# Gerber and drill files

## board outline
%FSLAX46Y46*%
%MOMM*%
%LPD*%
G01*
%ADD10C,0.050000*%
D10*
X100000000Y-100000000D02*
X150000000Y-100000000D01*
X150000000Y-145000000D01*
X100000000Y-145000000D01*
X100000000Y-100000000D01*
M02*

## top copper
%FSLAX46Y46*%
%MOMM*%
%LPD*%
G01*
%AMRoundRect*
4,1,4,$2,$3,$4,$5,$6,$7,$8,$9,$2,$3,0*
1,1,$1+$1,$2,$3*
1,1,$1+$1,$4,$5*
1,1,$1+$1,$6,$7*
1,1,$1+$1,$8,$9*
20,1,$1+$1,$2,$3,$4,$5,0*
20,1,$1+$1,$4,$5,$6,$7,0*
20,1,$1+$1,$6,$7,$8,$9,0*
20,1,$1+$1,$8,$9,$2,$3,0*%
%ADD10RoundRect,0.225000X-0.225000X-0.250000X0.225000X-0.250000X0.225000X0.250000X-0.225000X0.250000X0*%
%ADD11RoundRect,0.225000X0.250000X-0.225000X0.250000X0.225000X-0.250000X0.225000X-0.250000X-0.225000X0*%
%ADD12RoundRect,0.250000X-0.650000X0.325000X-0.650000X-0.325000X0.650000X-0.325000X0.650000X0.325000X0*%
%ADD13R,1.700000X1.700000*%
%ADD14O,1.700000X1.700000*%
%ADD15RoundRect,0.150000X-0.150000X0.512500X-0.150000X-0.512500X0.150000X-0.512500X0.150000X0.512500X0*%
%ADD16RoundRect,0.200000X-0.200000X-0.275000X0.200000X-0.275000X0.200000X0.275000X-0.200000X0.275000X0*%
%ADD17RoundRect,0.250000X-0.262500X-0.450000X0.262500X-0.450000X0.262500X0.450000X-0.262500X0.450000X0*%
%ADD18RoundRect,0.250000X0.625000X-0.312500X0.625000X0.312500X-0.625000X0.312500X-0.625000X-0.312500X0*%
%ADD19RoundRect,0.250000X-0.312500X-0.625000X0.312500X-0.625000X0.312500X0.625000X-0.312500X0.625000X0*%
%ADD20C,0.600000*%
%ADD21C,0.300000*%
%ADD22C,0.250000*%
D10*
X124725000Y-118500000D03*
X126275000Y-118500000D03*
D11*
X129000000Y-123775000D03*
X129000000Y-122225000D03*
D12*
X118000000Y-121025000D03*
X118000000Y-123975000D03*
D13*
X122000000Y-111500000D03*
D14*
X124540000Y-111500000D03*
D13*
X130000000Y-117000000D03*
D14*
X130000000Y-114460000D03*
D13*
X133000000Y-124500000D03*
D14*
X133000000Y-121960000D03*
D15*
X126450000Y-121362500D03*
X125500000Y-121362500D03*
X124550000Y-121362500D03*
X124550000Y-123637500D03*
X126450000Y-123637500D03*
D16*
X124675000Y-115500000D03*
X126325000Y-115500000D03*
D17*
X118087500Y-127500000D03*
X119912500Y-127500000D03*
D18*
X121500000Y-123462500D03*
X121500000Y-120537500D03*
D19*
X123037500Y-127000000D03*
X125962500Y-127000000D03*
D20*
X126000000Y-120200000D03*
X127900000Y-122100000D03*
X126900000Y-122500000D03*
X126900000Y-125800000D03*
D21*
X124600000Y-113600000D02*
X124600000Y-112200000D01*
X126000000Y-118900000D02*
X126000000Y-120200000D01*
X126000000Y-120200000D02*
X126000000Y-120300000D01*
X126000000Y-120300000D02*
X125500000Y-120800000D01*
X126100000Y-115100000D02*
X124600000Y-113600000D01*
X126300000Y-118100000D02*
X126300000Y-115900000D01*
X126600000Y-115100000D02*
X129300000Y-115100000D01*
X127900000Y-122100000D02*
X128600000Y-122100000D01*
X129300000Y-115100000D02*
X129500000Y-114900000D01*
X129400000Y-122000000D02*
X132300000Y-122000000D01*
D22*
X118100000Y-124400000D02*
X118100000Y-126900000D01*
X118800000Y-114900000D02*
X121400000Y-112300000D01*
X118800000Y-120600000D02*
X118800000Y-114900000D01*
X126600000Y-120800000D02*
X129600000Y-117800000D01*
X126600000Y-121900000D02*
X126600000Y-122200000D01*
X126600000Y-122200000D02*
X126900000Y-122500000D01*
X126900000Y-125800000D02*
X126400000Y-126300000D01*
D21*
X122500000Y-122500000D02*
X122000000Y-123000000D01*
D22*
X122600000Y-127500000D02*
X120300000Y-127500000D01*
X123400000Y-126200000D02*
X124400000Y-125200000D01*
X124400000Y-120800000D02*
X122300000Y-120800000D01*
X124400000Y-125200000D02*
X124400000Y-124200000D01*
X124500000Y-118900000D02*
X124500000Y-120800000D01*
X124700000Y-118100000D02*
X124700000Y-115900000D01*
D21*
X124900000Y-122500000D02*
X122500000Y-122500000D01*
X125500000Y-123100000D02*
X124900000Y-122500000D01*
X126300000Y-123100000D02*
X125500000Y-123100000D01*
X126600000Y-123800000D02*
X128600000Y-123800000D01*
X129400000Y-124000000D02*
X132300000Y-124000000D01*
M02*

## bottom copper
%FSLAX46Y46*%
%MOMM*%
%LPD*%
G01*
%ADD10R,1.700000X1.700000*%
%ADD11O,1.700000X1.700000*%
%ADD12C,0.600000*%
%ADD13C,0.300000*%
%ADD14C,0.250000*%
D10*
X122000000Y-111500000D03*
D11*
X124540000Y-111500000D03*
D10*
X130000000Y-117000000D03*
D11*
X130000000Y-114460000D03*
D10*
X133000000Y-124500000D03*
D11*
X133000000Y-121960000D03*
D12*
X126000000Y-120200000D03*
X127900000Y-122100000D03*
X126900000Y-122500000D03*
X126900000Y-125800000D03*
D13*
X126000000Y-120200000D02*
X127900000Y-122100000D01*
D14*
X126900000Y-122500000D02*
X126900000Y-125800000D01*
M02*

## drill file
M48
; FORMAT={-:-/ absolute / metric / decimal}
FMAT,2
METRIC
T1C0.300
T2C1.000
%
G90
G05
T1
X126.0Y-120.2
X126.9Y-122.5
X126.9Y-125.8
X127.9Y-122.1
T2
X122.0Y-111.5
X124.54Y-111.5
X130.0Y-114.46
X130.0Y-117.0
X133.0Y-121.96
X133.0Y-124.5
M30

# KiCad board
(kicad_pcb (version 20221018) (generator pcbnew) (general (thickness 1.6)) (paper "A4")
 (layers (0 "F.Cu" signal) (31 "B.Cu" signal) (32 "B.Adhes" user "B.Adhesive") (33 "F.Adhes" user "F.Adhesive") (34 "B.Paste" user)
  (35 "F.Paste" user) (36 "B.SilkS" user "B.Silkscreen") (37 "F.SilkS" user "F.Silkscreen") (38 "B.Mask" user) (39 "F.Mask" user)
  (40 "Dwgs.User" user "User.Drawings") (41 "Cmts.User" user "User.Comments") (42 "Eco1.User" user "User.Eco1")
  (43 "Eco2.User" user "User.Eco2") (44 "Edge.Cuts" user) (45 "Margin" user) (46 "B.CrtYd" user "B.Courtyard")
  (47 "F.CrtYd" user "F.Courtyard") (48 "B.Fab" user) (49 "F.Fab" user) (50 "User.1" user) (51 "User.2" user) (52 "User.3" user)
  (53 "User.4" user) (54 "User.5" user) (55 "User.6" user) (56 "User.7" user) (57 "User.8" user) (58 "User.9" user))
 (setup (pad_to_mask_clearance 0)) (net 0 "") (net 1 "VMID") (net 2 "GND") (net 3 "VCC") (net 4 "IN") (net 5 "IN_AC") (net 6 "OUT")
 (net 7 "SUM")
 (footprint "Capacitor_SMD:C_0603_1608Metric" (layer "F.Cu") (at 125.5 118.5)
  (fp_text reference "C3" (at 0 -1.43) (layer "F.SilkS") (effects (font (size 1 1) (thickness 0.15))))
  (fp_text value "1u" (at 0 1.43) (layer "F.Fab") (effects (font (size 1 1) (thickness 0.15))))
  (pad "1" smd roundrect (at -0.775 0) (size 0.9 0.95) (layers "F.Cu" "F.Paste" "F.Mask") (roundrect_rratio 0.25) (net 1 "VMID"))
  (pad "2" smd roundrect (at 0.775 0) (size 0.9 0.95) (layers "F.Cu" "F.Paste" "F.Mask") (roundrect_rratio 0.25) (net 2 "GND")))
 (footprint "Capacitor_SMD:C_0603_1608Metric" (layer "F.Cu") (at 129 123 90)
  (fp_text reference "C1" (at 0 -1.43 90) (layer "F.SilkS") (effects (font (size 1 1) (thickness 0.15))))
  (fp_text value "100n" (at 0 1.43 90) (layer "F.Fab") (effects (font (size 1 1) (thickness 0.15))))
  (pad "1" smd roundrect (at -0.775 0 90) (size 0.9 0.95) (layers "F.Cu" "F.Paste" "F.Mask") (roundrect_rratio 0.25) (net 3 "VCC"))
  (pad "2" smd roundrect (at 0.775 0 90) (size 0.9 0.95) (layers "F.Cu" "F.Paste" "F.Mask") (roundrect_rratio 0.25) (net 2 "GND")))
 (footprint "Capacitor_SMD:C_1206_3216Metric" (layer "F.Cu") (at 118 122.5 -90)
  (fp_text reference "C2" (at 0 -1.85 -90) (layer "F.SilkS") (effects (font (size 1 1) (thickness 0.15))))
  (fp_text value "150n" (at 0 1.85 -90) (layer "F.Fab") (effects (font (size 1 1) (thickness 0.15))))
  (pad "1" smd roundrect (at -1.475 0 270) (size 1.15 1.8) (layers "F.Cu" "F.Paste" "F.Mask") (roundrect_rratio 0.217391) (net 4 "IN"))
  (pad "2" smd roundrect (at 1.475 0 270) (size 1.15 1.8) (layers "F.Cu" "F.Paste" "F.Mask") (roundrect_rratio 0.217391) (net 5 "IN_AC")))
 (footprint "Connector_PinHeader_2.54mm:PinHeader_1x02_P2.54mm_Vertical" (layer "F.Cu") (at 122 111.5 90)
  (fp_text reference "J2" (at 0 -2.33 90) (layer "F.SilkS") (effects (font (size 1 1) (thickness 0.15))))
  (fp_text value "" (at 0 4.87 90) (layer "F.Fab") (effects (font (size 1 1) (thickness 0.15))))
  (pad "1" thru_hole rect (at 0 0 90) (size 1.7 1.7) (drill 1) (layers "*.Cu" "*.Mask") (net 4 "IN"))
  (pad "2" thru_hole oval (at 0 2.54 90) (size 1.7 1.7) (drill 1) (layers "*.Cu" "*.Mask") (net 2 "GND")))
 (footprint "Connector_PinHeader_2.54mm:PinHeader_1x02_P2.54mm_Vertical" (layer "F.Cu") (at 130 117 180)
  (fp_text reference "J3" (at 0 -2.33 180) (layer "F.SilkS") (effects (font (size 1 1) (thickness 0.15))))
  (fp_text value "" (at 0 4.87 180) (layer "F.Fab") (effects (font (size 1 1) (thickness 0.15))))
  (pad "1" thru_hole rect (at 0 0 180) (size 1.7 1.7) (drill 1) (layers "*.Cu" "*.Mask") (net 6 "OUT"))
  (pad "2" thru_hole oval (at 0 2.54 180) (size 1.7 1.7) (drill 1) (layers "*.Cu" "*.Mask") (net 2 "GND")))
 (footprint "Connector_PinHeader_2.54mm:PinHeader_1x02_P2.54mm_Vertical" (layer "F.Cu") (at 133 124.5 180)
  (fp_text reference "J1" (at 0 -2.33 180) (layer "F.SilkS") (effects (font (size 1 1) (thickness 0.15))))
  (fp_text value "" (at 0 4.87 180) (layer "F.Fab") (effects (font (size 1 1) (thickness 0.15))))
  (pad "1" thru_hole rect (at 0 0 180) (size 1.7 1.7) (drill 1) (layers "*.Cu" "*.Mask") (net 3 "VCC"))
  (pad "2" thru_hole oval (at 0 2.54 180) (size 1.7 1.7) (drill 1) (layers "*.Cu" "*.Mask") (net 2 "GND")))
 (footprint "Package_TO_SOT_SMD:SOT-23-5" (layer "F.Cu") (at 125.5 122.5 -90)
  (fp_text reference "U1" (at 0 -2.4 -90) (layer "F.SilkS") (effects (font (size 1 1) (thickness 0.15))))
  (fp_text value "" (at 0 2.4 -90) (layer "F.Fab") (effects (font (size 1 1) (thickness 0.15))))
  (pad "1" smd roundrect (at -1.1375 -0.95 270) (size 1.325 0.6) (layers "F.Cu" "F.Paste" "F.Mask") (roundrect_rratio 0.25) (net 6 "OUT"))
  (pad "2" smd roundrect (at -1.1375 0 270) (size 1.325 0.6) (layers "F.Cu" "F.Paste" "F.Mask") (roundrect_rratio 0.25) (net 2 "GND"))
  (pad "3" smd roundrect (at -1.1375 0.95 270) (size 1.325 0.6) (layers "F.Cu" "F.Paste" "F.Mask") (roundrect_rratio 0.25) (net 1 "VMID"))
  (pad "4" smd roundrect (at 1.1375 0.95 270) (size 1.325 0.6) (layers "F.Cu" "F.Paste" "F.Mask") (roundrect_rratio 0.25) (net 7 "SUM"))
  (pad "5" smd roundrect (at 1.1375 -0.95 270) (size 1.325 0.6) (layers "F.Cu" "F.Paste" "F.Mask") (roundrect_rratio 0.25) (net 3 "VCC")))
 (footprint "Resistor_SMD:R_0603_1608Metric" (layer "F.Cu") (at 125.5 115.5)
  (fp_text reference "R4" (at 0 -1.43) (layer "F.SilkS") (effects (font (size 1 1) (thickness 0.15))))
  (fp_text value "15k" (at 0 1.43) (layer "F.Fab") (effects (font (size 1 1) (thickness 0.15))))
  (pad "1" smd roundrect (at -0.825 0) (size 0.8 0.95) (layers "F.Cu" "F.Paste" "F.Mask") (roundrect_rratio 0.25) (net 1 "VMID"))
  (pad "2" smd roundrect (at 0.825 0) (size 0.8 0.95) (layers "F.Cu" "F.Paste" "F.Mask") (roundrect_rratio 0.25) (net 2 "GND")))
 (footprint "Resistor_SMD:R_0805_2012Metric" (layer "F.Cu") (at 119 127.5)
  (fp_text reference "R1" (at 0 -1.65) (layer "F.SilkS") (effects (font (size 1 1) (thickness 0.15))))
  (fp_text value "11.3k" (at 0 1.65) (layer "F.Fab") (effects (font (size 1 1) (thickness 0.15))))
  (pad "1" smd roundrect (at -0.9125 0) (size 1.025 1.4) (layers "F.Cu" "F.Paste" "F.Mask") (roundrect_rratio 0.243902) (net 5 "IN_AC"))
  (pad "2" smd roundrect (at 0.9125 0) (size 1.025 1.4) (layers "F.Cu" "F.Paste" "F.Mask") (roundrect_rratio 0.243902) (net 7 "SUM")))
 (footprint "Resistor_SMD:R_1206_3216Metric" (layer "F.Cu") (at 121.5 122 90)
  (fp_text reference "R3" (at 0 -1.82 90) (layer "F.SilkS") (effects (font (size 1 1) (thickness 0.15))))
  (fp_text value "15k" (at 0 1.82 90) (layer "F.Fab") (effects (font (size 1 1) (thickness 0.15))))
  (pad "1" smd roundrect (at -1.4625 0 90) (size 1.125 1.75) (layers "F.Cu" "F.Paste" "F.Mask") (roundrect_rratio 0.222222) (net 3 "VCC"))
  (pad "2" smd roundrect (at 1.4625 0 90) (size 1.125 1.75) (layers "F.Cu" "F.Paste" "F.Mask") (roundrect_rratio 0.222222) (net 1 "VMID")))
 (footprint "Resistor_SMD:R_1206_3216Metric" (layer "F.Cu") (at 124.5 127)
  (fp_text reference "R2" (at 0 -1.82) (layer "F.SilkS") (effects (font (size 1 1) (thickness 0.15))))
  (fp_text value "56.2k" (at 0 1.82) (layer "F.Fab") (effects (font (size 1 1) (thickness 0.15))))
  (pad "1" smd roundrect (at -1.4625 0) (size 1.125 1.75) (layers "F.Cu" "F.Paste" "F.Mask") (roundrect_rratio 0.222222) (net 7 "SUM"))
  (pad "2" smd roundrect (at 1.4625 0) (size 1.125 1.75) (layers "F.Cu" "F.Paste" "F.Mask") (roundrect_rratio 0.222222) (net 6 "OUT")))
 (gr_rect (start 100 100) (end 150 145) (stroke (width 0.05) (type default)) (fill none) (layer "Edge.Cuts"))
 (segment (start 124.6 113.6) (end 124.6 112.2) (width 0.3) (layer "F.Cu") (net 2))
 (segment (start 126 118.9) (end 126 120.2) (width 0.3) (layer "F.Cu") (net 2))
 (segment (start 126 120.2) (end 126 120.3) (width 0.3) (layer "F.Cu") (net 2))
 (segment (start 126 120.3) (end 125.5 120.8) (width 0.3) (layer "F.Cu") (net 2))
 (segment (start 126.1 115.1) (end 124.6 113.6) (width 0.3) (layer "F.Cu") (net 2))
 (segment (start 126.3 118.1) (end 126.3 115.9) (width 0.3) (layer "F.Cu") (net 2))
 (segment (start 126.6 115.1) (end 129.3 115.1) (width 0.3) (layer "F.Cu") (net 2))
 (segment (start 127.9 122.1) (end 128.6 122.1) (width 0.3) (layer "F.Cu") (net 2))
 (segment (start 129.3 115.1) (end 129.5 114.9) (width 0.3) (layer "F.Cu") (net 2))
 (segment (start 129.4 122) (end 132.3 122) (width 0.3) (layer "F.Cu") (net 2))
 (via (at 126 120.2) (size 0.6) (drill 0.3) (layers "F.Cu" "B.Cu") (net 2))
 (via (at 127.9 122.1) (size 0.6) (drill 0.3) (layers "F.Cu" "B.Cu") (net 2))
 (segment (start 118.1 124.4) (end 118.1 126.9) (width 0.25) (layer "F.Cu") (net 5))
 (segment (start 118.8 114.9) (end 121.4 112.3) (width 0.25) (layer "F.Cu") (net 4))
 (segment (start 118.8 120.6) (end 118.8 114.9) (width 0.25) (layer "F.Cu") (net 4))
 (segment (start 126 120.2) (end 127.9 122.1) (width 0.3) (layer "B.Cu") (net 2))
 (segment (start 126.6 120.8) (end 129.6 117.8) (width 0.25) (layer "F.Cu") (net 6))
 (segment (start 126.6 121.9) (end 126.6 122.2) (width 0.25) (layer "F.Cu") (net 6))
 (segment (start 126.6 122.2) (end 126.9 122.5) (width 0.25) (layer "F.Cu") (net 6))
 (segment (start 126.9 125.8) (end 126.4 126.3) (width 0.25) (layer "F.Cu") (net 6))
 (via (at 126.9 122.5) (size 0.6) (drill 0.3) (layers "F.Cu" "B.Cu") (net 6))
 (via (at 126.9 125.8) (size 0.6) (drill 0.3) (layers "F.Cu" "B.Cu") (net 6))
 (segment (start 122.5 122.5) (end 122 123) (width 0.3) (layer "F.Cu") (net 3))
 (segment (start 122.6 127.5) (end 120.3 127.5) (width 0.25) (layer "F.Cu") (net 7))
 (segment (start 123.4 126.2) (end 124.4 125.2) (width 0.25) (layer "F.Cu") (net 7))
 (segment (start 124.4 120.8) (end 122.3 120.8) (width 0.25) (layer "F.Cu") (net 1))
 (segment (start 124.4 125.2) (end 124.4 124.2) (width 0.25) (layer "F.Cu") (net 7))
 (segment (start 124.5 118.9) (end 124.5 120.8) (width 0.25) (layer "F.Cu") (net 1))
 (segment (start 124.7 118.1) (end 124.7 115.9) (width 0.25) (layer "F.Cu") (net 1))
 (segment (start 124.9 122.5) (end 122.5 122.5) (width 0.3) (layer "F.Cu") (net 3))
 (segment (start 125.5 123.1) (end 124.9 122.5) (width 0.3) (layer "F.Cu") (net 3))
 (segment (start 126.3 123.1) (end 125.5 123.1) (width 0.3) (layer "F.Cu") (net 3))
 (segment (start 126.6 123.8) (end 128.6 123.8) (width 0.3) (layer "F.Cu") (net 3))
 (segment (start 126.9 122.5) (end 126.9 125.8) (width 0.25) (layer "B.Cu") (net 6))
 (segment (start 129.4 124) (end 132.3 124) (width 0.3) (layer "F.Cu") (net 3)))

